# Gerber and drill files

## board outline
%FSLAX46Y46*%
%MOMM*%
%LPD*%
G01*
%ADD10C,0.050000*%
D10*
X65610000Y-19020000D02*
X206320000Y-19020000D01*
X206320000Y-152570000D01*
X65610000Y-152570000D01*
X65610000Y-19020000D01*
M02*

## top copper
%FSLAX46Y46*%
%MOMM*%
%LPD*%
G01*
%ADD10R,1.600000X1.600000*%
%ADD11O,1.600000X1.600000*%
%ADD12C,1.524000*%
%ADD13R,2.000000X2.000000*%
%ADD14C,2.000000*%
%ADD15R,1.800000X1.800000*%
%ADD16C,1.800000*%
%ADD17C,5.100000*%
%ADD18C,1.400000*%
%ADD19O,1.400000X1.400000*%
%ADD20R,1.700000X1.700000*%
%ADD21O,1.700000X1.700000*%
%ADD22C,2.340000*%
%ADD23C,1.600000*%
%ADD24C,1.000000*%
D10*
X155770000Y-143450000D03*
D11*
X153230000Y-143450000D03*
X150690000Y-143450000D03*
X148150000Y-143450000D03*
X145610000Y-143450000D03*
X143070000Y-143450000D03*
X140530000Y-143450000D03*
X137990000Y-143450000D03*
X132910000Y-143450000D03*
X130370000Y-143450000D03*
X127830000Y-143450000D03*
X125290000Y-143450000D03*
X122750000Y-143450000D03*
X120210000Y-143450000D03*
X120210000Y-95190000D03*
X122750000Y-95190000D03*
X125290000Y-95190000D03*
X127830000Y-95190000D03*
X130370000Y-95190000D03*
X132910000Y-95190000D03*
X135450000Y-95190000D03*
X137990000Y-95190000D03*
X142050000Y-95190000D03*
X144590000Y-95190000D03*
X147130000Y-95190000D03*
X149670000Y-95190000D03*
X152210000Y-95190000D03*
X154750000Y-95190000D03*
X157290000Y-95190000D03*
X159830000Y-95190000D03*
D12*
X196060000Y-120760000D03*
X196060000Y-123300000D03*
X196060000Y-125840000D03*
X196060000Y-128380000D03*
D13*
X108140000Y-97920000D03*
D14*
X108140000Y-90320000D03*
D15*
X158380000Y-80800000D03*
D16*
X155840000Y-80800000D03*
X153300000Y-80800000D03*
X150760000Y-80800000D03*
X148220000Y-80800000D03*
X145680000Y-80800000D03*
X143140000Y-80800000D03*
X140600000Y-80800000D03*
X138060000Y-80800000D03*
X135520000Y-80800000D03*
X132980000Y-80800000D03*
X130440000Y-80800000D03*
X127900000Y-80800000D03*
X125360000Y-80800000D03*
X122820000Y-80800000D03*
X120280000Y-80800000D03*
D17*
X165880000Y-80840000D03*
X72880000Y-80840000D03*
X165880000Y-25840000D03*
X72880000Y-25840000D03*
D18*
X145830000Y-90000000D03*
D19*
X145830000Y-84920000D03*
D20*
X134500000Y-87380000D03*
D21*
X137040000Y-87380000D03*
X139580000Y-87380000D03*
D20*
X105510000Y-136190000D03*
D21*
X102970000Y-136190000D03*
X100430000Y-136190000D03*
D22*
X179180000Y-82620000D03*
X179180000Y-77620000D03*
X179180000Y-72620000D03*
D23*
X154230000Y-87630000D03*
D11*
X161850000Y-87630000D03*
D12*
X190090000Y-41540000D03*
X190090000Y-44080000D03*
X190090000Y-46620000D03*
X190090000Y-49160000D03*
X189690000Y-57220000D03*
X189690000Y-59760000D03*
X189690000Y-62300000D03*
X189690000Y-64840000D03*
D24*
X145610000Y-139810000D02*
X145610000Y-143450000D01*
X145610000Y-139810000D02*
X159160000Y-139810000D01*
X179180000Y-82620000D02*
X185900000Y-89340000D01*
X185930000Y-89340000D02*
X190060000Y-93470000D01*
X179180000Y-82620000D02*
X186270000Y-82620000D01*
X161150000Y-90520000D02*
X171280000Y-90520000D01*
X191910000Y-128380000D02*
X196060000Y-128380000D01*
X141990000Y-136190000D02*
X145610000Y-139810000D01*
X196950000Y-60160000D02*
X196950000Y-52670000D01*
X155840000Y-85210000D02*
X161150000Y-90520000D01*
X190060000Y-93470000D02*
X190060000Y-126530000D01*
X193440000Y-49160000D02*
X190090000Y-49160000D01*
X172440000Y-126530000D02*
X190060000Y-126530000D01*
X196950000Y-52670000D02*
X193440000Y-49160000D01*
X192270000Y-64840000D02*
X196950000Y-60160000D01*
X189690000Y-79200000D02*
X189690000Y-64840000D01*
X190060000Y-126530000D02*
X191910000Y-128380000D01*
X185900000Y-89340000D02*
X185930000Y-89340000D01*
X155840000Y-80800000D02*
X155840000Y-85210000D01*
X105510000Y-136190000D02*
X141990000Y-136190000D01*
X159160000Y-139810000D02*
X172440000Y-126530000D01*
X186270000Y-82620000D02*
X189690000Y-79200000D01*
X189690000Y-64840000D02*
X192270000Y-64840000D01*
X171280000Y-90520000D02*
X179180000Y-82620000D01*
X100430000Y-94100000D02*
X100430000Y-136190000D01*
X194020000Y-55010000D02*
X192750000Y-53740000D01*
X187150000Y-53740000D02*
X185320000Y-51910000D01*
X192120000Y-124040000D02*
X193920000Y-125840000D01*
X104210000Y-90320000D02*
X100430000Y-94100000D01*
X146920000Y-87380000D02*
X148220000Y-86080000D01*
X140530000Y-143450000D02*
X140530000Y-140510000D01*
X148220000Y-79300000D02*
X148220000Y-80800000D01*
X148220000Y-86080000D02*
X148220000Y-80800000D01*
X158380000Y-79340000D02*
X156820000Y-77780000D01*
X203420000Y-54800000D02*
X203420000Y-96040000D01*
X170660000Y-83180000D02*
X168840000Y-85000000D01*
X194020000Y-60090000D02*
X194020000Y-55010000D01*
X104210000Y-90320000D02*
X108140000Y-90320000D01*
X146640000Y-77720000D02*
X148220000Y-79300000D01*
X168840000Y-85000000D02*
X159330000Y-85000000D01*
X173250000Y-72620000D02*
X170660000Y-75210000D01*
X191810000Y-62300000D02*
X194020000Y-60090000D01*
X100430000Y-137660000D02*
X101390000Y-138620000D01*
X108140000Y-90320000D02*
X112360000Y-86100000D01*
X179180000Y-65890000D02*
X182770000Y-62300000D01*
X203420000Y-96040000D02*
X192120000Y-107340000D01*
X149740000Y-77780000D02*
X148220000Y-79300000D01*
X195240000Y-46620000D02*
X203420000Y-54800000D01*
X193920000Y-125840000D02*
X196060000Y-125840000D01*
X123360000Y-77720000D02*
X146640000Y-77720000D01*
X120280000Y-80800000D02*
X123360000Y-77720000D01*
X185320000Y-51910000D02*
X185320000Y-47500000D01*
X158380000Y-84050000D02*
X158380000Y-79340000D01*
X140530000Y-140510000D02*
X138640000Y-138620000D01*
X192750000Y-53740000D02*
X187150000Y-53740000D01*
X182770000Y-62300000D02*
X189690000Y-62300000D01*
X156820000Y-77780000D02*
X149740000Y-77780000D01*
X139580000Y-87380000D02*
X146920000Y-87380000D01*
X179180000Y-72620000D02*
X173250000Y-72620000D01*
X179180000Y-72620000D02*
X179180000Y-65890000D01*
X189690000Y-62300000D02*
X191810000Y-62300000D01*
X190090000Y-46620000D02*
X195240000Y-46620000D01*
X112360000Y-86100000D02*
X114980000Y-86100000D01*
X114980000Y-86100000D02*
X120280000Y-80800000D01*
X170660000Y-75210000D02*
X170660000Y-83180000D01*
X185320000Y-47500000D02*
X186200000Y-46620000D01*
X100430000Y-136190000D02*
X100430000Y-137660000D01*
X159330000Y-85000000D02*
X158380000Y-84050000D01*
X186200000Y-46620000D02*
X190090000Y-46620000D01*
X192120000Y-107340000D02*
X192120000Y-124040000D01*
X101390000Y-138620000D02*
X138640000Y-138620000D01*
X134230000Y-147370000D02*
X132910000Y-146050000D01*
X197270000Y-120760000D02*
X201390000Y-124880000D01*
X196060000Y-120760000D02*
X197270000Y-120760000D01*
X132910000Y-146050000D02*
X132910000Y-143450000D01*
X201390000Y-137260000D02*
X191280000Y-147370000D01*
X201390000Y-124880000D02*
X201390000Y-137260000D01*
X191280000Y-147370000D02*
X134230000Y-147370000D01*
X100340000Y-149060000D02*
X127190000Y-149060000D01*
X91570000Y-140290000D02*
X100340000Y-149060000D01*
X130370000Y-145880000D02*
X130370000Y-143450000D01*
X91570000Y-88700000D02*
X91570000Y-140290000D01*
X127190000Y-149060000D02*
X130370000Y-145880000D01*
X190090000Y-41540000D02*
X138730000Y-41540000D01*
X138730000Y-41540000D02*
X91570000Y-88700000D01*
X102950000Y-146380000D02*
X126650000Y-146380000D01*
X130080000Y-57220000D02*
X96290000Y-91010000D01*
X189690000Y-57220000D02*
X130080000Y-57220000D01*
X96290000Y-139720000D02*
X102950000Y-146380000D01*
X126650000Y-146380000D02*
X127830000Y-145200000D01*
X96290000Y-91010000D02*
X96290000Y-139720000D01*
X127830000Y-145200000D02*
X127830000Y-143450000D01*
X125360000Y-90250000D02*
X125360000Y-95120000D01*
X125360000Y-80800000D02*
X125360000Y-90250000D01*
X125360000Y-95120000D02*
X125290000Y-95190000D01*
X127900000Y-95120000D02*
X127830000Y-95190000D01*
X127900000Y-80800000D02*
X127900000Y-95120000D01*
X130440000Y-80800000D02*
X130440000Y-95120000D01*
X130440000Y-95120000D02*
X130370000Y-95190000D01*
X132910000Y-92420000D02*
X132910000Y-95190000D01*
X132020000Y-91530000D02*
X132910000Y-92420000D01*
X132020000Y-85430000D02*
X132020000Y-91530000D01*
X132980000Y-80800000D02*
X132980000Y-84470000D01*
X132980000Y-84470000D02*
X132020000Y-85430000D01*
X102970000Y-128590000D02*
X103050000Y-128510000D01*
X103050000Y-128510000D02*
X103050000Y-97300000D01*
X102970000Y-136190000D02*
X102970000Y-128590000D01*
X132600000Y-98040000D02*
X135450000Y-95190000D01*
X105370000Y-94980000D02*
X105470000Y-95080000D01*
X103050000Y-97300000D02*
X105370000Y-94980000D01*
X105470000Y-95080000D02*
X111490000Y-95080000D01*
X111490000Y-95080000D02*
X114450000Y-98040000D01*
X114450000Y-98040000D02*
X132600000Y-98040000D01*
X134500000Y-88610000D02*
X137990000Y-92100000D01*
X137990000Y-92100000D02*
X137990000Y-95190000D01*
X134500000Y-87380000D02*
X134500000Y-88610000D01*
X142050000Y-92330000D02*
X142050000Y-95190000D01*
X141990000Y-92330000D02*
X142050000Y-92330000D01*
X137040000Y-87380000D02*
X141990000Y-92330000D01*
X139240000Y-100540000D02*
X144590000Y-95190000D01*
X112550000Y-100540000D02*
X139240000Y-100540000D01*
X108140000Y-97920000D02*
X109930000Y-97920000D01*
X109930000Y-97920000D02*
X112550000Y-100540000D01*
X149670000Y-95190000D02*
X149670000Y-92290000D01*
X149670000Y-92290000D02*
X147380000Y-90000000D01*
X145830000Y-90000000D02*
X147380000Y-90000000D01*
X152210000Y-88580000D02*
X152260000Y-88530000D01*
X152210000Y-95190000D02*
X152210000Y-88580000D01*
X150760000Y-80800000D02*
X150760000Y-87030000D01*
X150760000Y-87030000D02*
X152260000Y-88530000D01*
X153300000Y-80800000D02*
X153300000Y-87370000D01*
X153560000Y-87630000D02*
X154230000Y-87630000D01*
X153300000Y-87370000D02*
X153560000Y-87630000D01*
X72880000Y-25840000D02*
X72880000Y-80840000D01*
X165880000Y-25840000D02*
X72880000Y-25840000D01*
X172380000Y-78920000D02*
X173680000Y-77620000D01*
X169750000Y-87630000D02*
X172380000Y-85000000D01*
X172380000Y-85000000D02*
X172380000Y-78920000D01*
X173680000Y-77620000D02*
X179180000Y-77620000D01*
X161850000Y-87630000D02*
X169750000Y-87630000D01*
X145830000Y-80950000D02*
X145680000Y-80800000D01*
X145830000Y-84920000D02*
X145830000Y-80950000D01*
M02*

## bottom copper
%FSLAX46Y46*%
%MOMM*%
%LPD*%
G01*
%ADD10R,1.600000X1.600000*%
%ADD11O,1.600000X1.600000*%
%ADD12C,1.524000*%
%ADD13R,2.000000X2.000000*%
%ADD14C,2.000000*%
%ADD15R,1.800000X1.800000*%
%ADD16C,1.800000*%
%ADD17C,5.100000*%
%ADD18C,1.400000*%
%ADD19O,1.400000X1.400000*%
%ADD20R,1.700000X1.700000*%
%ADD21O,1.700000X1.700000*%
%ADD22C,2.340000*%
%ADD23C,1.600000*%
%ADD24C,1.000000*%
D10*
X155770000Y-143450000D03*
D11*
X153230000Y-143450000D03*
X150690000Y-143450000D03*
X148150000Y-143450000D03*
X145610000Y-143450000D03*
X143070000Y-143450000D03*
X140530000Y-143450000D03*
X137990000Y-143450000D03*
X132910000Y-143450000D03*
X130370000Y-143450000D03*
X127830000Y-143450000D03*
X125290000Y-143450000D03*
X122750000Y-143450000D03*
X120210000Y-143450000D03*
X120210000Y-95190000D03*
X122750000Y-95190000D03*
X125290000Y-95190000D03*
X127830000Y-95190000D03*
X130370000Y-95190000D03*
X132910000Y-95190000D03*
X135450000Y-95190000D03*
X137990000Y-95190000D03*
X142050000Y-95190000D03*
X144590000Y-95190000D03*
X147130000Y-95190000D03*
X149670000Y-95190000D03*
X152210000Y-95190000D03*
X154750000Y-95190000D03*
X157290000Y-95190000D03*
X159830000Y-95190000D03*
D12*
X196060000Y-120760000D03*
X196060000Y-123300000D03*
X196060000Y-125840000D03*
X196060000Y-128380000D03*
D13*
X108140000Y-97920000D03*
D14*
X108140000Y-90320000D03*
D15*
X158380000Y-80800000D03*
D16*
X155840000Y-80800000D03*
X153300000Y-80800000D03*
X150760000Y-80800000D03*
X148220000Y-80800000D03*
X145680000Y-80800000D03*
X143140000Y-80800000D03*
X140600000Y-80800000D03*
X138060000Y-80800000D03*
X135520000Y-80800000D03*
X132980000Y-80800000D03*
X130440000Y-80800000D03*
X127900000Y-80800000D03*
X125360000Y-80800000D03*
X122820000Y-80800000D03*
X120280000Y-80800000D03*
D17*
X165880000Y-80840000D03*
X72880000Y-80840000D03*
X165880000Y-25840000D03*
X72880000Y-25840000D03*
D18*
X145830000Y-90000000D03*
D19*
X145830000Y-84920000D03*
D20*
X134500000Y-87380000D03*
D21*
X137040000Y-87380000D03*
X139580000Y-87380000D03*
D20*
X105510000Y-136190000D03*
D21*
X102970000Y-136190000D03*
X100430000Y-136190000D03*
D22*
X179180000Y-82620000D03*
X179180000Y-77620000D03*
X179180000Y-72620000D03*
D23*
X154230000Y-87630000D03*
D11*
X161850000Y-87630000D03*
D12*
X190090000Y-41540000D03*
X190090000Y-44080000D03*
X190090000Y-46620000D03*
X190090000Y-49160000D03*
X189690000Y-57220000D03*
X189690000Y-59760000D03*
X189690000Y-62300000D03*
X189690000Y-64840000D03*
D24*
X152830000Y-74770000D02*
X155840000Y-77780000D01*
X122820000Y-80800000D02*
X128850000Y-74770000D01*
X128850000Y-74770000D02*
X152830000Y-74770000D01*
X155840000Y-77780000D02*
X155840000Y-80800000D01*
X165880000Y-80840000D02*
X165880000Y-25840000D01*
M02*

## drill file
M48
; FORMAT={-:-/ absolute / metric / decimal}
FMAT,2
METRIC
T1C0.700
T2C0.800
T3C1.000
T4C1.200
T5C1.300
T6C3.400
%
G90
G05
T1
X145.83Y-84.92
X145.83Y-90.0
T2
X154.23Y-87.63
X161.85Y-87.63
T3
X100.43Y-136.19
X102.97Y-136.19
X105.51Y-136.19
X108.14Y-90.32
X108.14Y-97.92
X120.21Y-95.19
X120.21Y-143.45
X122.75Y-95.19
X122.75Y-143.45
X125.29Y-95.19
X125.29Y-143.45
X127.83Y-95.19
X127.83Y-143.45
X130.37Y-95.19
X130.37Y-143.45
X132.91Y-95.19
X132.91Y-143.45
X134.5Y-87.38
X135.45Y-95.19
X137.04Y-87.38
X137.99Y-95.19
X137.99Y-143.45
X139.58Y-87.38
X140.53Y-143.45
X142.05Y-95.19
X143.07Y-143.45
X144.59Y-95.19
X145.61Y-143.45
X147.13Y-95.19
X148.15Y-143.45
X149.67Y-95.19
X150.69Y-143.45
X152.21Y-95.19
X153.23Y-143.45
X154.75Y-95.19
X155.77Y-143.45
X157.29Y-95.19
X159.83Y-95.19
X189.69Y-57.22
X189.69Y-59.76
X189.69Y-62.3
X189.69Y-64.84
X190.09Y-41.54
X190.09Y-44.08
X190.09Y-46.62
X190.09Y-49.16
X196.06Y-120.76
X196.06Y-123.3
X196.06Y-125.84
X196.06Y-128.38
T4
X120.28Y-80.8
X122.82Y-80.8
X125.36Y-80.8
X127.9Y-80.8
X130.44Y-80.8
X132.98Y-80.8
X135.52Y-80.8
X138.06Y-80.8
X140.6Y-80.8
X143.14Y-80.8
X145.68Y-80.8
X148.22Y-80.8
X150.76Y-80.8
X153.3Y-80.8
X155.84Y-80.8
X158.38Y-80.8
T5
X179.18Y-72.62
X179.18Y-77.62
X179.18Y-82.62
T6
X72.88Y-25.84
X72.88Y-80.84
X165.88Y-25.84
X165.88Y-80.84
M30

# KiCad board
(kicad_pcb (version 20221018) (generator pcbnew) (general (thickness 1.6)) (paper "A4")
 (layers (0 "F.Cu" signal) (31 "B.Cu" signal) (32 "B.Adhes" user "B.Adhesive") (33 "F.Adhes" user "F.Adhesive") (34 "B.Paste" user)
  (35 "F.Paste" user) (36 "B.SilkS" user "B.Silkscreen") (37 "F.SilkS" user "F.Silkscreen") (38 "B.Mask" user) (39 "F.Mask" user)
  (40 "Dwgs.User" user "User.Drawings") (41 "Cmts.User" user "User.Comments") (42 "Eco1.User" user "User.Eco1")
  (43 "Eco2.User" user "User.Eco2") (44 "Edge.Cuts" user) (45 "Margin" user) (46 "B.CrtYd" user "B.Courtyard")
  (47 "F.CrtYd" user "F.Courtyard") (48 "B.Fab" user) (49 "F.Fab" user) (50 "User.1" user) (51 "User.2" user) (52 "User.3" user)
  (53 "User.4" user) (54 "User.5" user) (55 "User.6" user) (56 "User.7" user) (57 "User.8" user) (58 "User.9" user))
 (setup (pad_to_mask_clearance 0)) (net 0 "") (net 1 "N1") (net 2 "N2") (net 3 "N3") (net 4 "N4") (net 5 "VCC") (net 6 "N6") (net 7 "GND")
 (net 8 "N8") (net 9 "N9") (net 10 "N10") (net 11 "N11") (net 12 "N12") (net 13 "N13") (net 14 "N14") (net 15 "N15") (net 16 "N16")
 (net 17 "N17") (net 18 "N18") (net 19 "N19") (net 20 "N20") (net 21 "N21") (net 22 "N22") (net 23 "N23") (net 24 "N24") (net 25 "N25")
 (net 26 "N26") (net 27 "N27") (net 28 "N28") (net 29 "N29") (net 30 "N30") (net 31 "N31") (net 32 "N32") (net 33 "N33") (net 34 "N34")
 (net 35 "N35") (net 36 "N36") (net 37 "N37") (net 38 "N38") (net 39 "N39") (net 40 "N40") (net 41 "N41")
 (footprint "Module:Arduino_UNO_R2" (layer "F.Cu") (at 155.77 143.45 180)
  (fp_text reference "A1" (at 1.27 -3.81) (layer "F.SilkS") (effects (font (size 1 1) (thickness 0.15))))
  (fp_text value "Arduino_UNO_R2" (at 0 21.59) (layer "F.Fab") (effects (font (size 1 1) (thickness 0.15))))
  (pad "1" thru_hole rect (at 0 0 270) (size 1.6 1.6) (drill 1) (layers "*.Cu" "*.Mask") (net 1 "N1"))
  (pad "2" thru_hole oval (at 2.54 0 270) (size 1.6 1.6) (drill 1) (layers "*.Cu" "*.Mask") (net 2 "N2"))
  (pad "3" thru_hole oval (at 5.08 0 270) (size 1.6 1.6) (drill 1) (layers "*.Cu" "*.Mask") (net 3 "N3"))
  (pad "4" thru_hole oval (at 7.62 0 270) (size 1.6 1.6) (drill 1) (layers "*.Cu" "*.Mask") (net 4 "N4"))
  (pad "5" thru_hole oval (at 10.16 0 270) (size 1.6 1.6) (drill 1) (layers "*.Cu" "*.Mask") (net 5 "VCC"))
  (pad "6" thru_hole oval (at 12.7 0 270) (size 1.6 1.6) (drill 1) (layers "*.Cu" "*.Mask") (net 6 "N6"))
  (pad "7" thru_hole oval (at 15.24 0 270) (size 1.6 1.6) (drill 1) (layers "*.Cu" "*.Mask") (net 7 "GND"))
  (pad "8" thru_hole oval (at 17.78 0 270) (size 1.6 1.6) (drill 1) (layers "*.Cu" "*.Mask") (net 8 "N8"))
  (pad "9" thru_hole oval (at 22.86 0 270) (size 1.6 1.6) (drill 1) (layers "*.Cu" "*.Mask") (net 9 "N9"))
  (pad "10" thru_hole oval (at 25.4 0 270) (size 1.6 1.6) (drill 1) (layers "*.Cu" "*.Mask") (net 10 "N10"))
  (pad "11" thru_hole oval (at 27.94 0 270) (size 1.6 1.6) (drill 1) (layers "*.Cu" "*.Mask") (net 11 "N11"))
  (pad "12" thru_hole oval (at 30.48 0 270) (size 1.6 1.6) (drill 1) (layers "*.Cu" "*.Mask") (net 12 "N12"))
  (pad "13" thru_hole oval (at 33.02 0 270) (size 1.6 1.6) (drill 1) (layers "*.Cu" "*.Mask") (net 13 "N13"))
  (pad "14" thru_hole oval (at 35.56 0 270) (size 1.6 1.6) (drill 1) (layers "*.Cu" "*.Mask") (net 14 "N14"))
  (pad "15" thru_hole oval (at 35.56 48.26 270) (size 1.6 1.6) (drill 1) (layers "*.Cu" "*.Mask") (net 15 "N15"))
  (pad "16" thru_hole oval (at 33.02 48.26 270) (size 1.6 1.6) (drill 1) (layers "*.Cu" "*.Mask") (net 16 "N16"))
  (pad "17" thru_hole oval (at 30.48 48.26 270) (size 1.6 1.6) (drill 1) (layers "*.Cu" "*.Mask") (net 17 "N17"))
  (pad "18" thru_hole oval (at 27.94 48.26 270) (size 1.6 1.6) (drill 1) (layers "*.Cu" "*.Mask") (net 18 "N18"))
  (pad "19" thru_hole oval (at 25.4 48.26 270) (size 1.6 1.6) (drill 1) (layers "*.Cu" "*.Mask") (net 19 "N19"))
  (pad "20" thru_hole oval (at 22.86 48.26 270) (size 1.6 1.6) (drill 1) (layers "*.Cu" "*.Mask") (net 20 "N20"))
  (pad "21" thru_hole oval (at 20.32 48.26 270) (size 1.6 1.6) (drill 1) (layers "*.Cu" "*.Mask") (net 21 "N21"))
  (pad "22" thru_hole oval (at 17.78 48.26 270) (size 1.6 1.6) (drill 1) (layers "*.Cu" "*.Mask") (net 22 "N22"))
  (pad "23" thru_hole oval (at 13.72 48.26 270) (size 1.6 1.6) (drill 1) (layers "*.Cu" "*.Mask") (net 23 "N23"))
  (pad "24" thru_hole oval (at 11.18 48.26 270) (size 1.6 1.6) (drill 1) (layers "*.Cu" "*.Mask") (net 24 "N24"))
  (pad "25" thru_hole oval (at 8.64 48.26 270) (size 1.6 1.6) (drill 1) (layers "*.Cu" "*.Mask") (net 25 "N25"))
  (pad "26" thru_hole oval (at 6.1 48.26 270) (size 1.6 1.6) (drill 1) (layers "*.Cu" "*.Mask") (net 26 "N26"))
  (pad "27" thru_hole oval (at 3.56 48.26 270) (size 1.6 1.6) (drill 1) (layers "*.Cu" "*.Mask") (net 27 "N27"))
  (pad "28" thru_hole oval (at 1.02 48.26 270) (size 1.6 1.6) (drill 1) (layers "*.Cu" "*.Mask") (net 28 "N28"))
  (pad "29" thru_hole oval (at -1.52 48.26 270) (size 1.6 1.6) (drill 1) (layers "*.Cu" "*.Mask") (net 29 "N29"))
  (pad "30" thru_hole oval (at -4.06 48.26 270) (size 1.6 1.6) (drill 1) (layers "*.Cu" "*.Mask") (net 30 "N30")))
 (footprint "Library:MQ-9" (layer "F.Cu") (at 201.14 115.68)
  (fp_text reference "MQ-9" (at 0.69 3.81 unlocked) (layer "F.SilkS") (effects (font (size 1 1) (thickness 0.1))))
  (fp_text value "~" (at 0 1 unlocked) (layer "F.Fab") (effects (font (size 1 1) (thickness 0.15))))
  (pad "1" thru_hole circle (at -5.08 5.08) (size 1.524 1.524) (drill 1) (layers "*.Cu" "*.Mask") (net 9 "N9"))
  (pad "2" thru_hole circle (at -5.08 7.62) (size 1.524 1.524) (drill 1) (layers "*.Cu" "*.Mask") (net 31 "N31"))
  (pad "3" thru_hole circle (at -5.08 10.16) (size 1.524 1.524) (drill 1) (layers "*.Cu" "*.Mask") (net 7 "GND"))
  (pad "4" thru_hole circle (at -5.08 12.7) (size 1.524 1.524) (drill 1) (layers "*.Cu" "*.Mask") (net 5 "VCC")))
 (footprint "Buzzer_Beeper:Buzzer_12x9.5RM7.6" (layer "F.Cu") (at 108.14 97.92 90)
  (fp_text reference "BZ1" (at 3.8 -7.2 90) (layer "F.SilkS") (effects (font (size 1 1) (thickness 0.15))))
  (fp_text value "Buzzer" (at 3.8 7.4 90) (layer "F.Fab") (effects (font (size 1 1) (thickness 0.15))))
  (pad "1" thru_hole rect (at 0 0 90) (size 2 2) (drill 1) (layers "*.Cu" "*.Mask") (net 24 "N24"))
  (pad "2" thru_hole circle (at 7.6 0 90) (size 2 2) (drill 1) (layers "*.Cu" "*.Mask") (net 7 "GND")))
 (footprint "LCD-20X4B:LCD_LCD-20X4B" (layer "F.Cu") (at 119.38 53.34 180)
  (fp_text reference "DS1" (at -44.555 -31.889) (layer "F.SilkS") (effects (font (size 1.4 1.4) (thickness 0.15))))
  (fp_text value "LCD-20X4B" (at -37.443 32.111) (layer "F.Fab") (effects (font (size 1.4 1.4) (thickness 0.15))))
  (pad "1" thru_hole rect (at -39 -27.46 180) (size 1.8 1.8) (drill 1.2) (layers "*.Cu" "*.Mask") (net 7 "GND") (solder_mask_margin 0.102))
  (pad "2" thru_hole circle (at -36.46 -27.46 180) (size 1.8 1.8) (drill 1.2) (layers "*.Cu" "*.Mask") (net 5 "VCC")
   (solder_mask_margin 0.102))
  (pad "3" thru_hole circle (at -33.92 -27.46 180) (size 1.8 1.8) (drill 1.2) (layers "*.Cu" "*.Mask") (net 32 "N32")
   (solder_mask_margin 0.102))
  (pad "4" thru_hole circle (at -31.38 -27.46 180) (size 1.8 1.8) (drill 1.2) (layers "*.Cu" "*.Mask") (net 27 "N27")
   (solder_mask_margin 0.102))
  (pad "5" thru_hole circle (at -28.84 -27.46 180) (size 1.8 1.8) (drill 1.2) (layers "*.Cu" "*.Mask") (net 7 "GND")
   (solder_mask_margin 0.102))
  (pad "6" thru_hole circle (at -26.3 -27.46 180) (size 1.8 1.8) (drill 1.2) (layers "*.Cu" "*.Mask") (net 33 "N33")
   (solder_mask_margin 0.102))
  (pad "7" thru_hole circle (at -23.76 -27.46 180) (size 1.8 1.8) (drill 1.2) (layers "*.Cu" "*.Mask") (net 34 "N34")
   (solder_mask_margin 0.102))
  (pad "8" thru_hole circle (at -21.22 -27.46 180) (size 1.8 1.8) (drill 1.2) (layers "*.Cu" "*.Mask") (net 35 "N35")
   (solder_mask_margin 0.102))
  (pad "9" thru_hole circle (at -18.68 -27.46 180) (size 1.8 1.8) (drill 1.2) (layers "*.Cu" "*.Mask") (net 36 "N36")
   (solder_mask_margin 0.102))
  (pad "10" thru_hole circle (at -16.14 -27.46 180) (size 1.8 1.8) (drill 1.2) (layers "*.Cu" "*.Mask") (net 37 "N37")
   (solder_mask_margin 0.102))
  (pad "11" thru_hole circle (at -13.6 -27.46 180) (size 1.8 1.8) (drill 1.2) (layers "*.Cu" "*.Mask") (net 20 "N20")
   (solder_mask_margin 0.102))
  (pad "12" thru_hole circle (at -11.06 -27.46 180) (size 1.8 1.8) (drill 1.2) (layers "*.Cu" "*.Mask") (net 19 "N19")
   (solder_mask_margin 0.102))
  (pad "13" thru_hole circle (at -8.52 -27.46 180) (size 1.8 1.8) (drill 1.2) (layers "*.Cu" "*.Mask") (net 18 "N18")
   (solder_mask_margin 0.102))
  (pad "14" thru_hole circle (at -5.98 -27.46 180) (size 1.8 1.8) (drill 1.2) (layers "*.Cu" "*.Mask") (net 17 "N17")
   (solder_mask_margin 0.102))
  (pad "15" thru_hole circle (at -3.44 -27.46 180) (size 1.8 1.8) (drill 1.2) (layers "*.Cu" "*.Mask") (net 5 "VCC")
   (solder_mask_margin 0.102))
  (pad "16" thru_hole circle (at -0.9 -27.46 180) (size 1.8 1.8) (drill 1.2) (layers "*.Cu" "*.Mask") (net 7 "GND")
   (solder_mask_margin 0.102))
  (pad "S1" thru_hole circle (at -46.5 -27.5 180) (size 5.1 5.1) (drill 3.4) (layers "*.Cu" "*.Mask") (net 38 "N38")
   (solder_mask_margin 0.102))
  (pad "S2" thru_hole circle (at 46.5 -27.5 180) (size 5.1 5.1) (drill 3.4) (layers "*.Cu" "*.Mask") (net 38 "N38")
   (solder_mask_margin 0.102))
  (pad "S3" thru_hole circle (at -46.5 27.5 180) (size 5.1 5.1) (drill 3.4) (layers "*.Cu" "*.Mask") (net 38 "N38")
   (solder_mask_margin 0.102))
  (pad "S4" thru_hole circle (at 46.5 27.5 180) (size 5.1 5.1) (drill 3.4) (layers "*.Cu" "*.Mask") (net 38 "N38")
   (solder_mask_margin 0.102)))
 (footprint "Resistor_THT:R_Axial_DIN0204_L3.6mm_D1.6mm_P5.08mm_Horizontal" (layer "F.Cu") (at 145.83 90 90)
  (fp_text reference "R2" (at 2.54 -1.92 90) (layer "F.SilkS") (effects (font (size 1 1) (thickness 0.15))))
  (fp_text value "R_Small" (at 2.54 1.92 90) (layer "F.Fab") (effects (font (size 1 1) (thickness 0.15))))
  (pad "1" thru_hole circle (at 0 0 90) (size 1.4 1.4) (drill 0.7) (layers "*.Cu" "*.Mask") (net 26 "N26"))
  (pad "2" thru_hole oval (at 5.08 0 90) (size 1.4 1.4) (drill 0.7) (layers "*.Cu" "*.Mask") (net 33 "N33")))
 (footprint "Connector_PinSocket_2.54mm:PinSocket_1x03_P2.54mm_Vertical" (layer "F.Cu") (at 134.5 87.38 90)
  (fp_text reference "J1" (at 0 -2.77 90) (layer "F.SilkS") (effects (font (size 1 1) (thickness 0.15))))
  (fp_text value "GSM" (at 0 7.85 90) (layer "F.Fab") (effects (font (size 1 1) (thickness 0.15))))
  (pad "1" thru_hole rect (at 0 0 90) (size 1.7 1.7) (drill 1) (layers "*.Cu" "*.Mask") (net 22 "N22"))
  (pad "2" thru_hole oval (at 0 2.54 90) (size 1.7 1.7) (drill 1) (layers "*.Cu" "*.Mask") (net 23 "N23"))
  (pad "3" thru_hole oval (at 0 5.08 90) (size 1.7 1.7) (drill 1) (layers "*.Cu" "*.Mask") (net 7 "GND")))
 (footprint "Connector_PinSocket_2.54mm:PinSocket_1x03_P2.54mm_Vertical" (layer "F.Cu") (at 105.51 136.19 -90)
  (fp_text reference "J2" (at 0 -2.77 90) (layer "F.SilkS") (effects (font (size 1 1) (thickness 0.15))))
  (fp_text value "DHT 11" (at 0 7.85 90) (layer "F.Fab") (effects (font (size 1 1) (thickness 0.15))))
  (pad "1" thru_hole rect (at 0 0 270) (size 1.7 1.7) (drill 1) (layers "*.Cu" "*.Mask") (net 5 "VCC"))
  (pad "2" thru_hole oval (at 0 2.54 270) (size 1.7 1.7) (drill 1) (layers "*.Cu" "*.Mask") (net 21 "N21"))
  (pad "3" thru_hole oval (at 0 5.08 270) (size 1.7 1.7) (drill 1) (layers "*.Cu" "*.Mask") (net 7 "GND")))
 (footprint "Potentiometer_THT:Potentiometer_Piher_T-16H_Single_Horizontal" (layer "F.Cu") (at 179.18 82.62)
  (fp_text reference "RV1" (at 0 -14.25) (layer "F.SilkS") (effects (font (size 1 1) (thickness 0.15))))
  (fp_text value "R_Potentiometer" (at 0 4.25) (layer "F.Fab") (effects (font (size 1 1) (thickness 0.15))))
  (pad "1" thru_hole circle (at 0 0) (size 2.34 2.34) (drill 1.3) (layers "*.Cu" "*.Mask") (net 5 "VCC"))
  (pad "2" thru_hole circle (at 0 -5) (size 2.34 2.34) (drill 1.3) (layers "*.Cu" "*.Mask") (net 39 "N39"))
  (pad "3" thru_hole circle (at 0 -10) (size 2.34 2.34) (drill 1.3) (layers "*.Cu" "*.Mask") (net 7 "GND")))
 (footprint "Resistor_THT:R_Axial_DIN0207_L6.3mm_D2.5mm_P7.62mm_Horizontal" (layer "F.Cu") (at 154.23 87.63)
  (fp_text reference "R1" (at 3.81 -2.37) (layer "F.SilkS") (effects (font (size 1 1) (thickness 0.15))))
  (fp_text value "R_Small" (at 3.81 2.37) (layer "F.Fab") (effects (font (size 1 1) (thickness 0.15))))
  (pad "1" thru_hole circle (at 0 0) (size 1.6 1.6) (drill 0.8) (layers "*.Cu" "*.Mask") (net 32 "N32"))
  (pad "2" thru_hole oval (at 7.62 0) (size 1.6 1.6) (drill 0.8) (layers "*.Cu" "*.Mask") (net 39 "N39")))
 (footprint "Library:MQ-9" (layer "F.Cu") (at 195.17 36.46)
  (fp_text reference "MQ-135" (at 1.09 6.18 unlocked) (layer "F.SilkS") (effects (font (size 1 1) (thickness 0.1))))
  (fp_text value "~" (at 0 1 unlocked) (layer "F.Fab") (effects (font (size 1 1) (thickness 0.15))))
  (pad "1" thru_hole circle (at -5.08 5.08) (size 1.524 1.524) (drill 1) (layers "*.Cu" "*.Mask") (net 10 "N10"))
  (pad "2" thru_hole circle (at -5.08 7.62) (size 1.524 1.524) (drill 1) (layers "*.Cu" "*.Mask") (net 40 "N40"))
  (pad "3" thru_hole circle (at -5.08 10.16) (size 1.524 1.524) (drill 1) (layers "*.Cu" "*.Mask") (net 7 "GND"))
  (pad "4" thru_hole circle (at -5.08 12.7) (size 1.524 1.524) (drill 1) (layers "*.Cu" "*.Mask") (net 5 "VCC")))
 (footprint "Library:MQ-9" (layer "F.Cu") (at 194.77 52.14)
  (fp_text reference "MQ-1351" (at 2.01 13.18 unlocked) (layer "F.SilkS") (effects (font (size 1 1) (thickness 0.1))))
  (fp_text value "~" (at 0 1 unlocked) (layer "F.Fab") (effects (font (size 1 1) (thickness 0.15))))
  (pad "1" thru_hole circle (at -5.08 5.08) (size 1.524 1.524) (drill 1) (layers "*.Cu" "*.Mask") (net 11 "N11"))
  (pad "2" thru_hole circle (at -5.08 7.62) (size 1.524 1.524) (drill 1) (layers "*.Cu" "*.Mask") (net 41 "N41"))
  (pad "3" thru_hole circle (at -5.08 10.16) (size 1.524 1.524) (drill 1) (layers "*.Cu" "*.Mask") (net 7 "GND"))
  (pad "4" thru_hole circle (at -5.08 12.7) (size 1.524 1.524) (drill 1) (layers "*.Cu" "*.Mask") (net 5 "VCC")))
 (gr_rect (start 65.61 19.02) (end 206.32 152.57) (stroke (width 0.05) (type default)) (fill none) (layer "Edge.Cuts"))
 (segment (start 145.61 139.81) (end 145.61 143.45) (width 1) (layer "F.Cu") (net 5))
 (segment (start 145.61 139.81) (end 159.16 139.81) (width 1) (layer "F.Cu") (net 5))
 (segment (start 179.18 82.62) (end 185.9 89.34) (width 1) (layer "F.Cu") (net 5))
 (segment (start 185.93 89.34) (end 190.06 93.47) (width 1) (layer "F.Cu") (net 5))
 (segment (start 179.18 82.62) (end 186.27 82.62) (width 1) (layer "F.Cu") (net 5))
 (segment (start 161.15 90.52) (end 171.28 90.52) (width 1) (layer "F.Cu") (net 5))
 (segment (start 191.91 128.38) (end 196.06 128.38) (width 1) (layer "F.Cu") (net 5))
 (segment (start 141.99 136.19) (end 145.61 139.81) (width 1) (layer "F.Cu") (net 5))
 (segment (start 196.95 60.16) (end 196.95 52.67) (width 1) (layer "F.Cu") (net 5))
 (segment (start 155.84 85.21) (end 161.15 90.52) (width 1) (layer "F.Cu") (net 5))
 (segment (start 190.06 93.47) (end 190.06 126.53) (width 1) (layer "F.Cu") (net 5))
 (segment (start 193.44 49.16) (end 190.09 49.16) (width 1) (layer "F.Cu") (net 5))
 (segment (start 172.44 126.53) (end 190.06 126.53) (width 1) (layer "F.Cu") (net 5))
 (segment (start 196.95 52.67) (end 193.44 49.16) (width 1) (layer "F.Cu") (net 5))
 (segment (start 192.27 64.84) (end 196.95 60.16) (width 1) (layer "F.Cu") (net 5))
 (segment (start 189.69 79.2) (end 189.69 64.84) (width 1) (layer "F.Cu") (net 5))
 (segment (start 190.06 126.53) (end 191.91 128.38) (width 1) (layer "F.Cu") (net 5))
 (segment (start 185.9 89.34) (end 185.93 89.34) (width 1) (layer "F.Cu") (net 5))
 (segment (start 155.84 80.8) (end 155.84 85.21) (width 1) (layer "F.Cu") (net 5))
 (segment (start 105.51 136.19) (end 141.99 136.19) (width 1) (layer "F.Cu") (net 5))
 (segment (start 159.16 139.81) (end 172.44 126.53) (width 1) (layer "F.Cu") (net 5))
 (segment (start 186.27 82.62) (end 189.69 79.2) (width 1) (layer "F.Cu") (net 5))
 (segment (start 189.69 64.84) (end 192.27 64.84) (width 1) (layer "F.Cu") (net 5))
 (segment (start 171.28 90.52) (end 179.18 82.62) (width 1) (layer "F.Cu") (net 5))
 (segment (start 152.83 74.77) (end 155.84 77.78) (width 1) (layer "B.Cu") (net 5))
 (segment (start 122.82 80.8) (end 128.85 74.77) (width 1) (layer "B.Cu") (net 5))
 (segment (start 128.85 74.77) (end 152.83 74.77) (width 1) (layer "B.Cu") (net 5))
 (segment (start 155.84 77.78) (end 155.84 80.8) (width 1) (layer "B.Cu") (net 5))
 (segment (start 100.43 94.1) (end 100.43 136.19) (width 1) (layer "F.Cu") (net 7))
 (segment (start 194.02 55.01) (end 192.75 53.74) (width 1) (layer "F.Cu") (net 7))
 (segment (start 187.15 53.74) (end 185.32 51.91) (width 1) (layer "F.Cu") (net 7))
 (segment (start 192.12 124.04) (end 193.92 125.84) (width 1) (layer "F.Cu") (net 7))
 (segment (start 104.21 90.32) (end 100.43 94.1) (width 1) (layer "F.Cu") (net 7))
 (segment (start 146.92 87.38) (end 148.22 86.08) (width 1) (layer "F.Cu") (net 7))
 (segment (start 140.53 143.45) (end 140.53 140.51) (width 1) (layer "F.Cu") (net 7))
 (segment (start 148.22 79.3) (end 148.22 80.8) (width 1) (layer "F.Cu") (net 7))
 (segment (start 148.22 86.08) (end 148.22 80.8) (width 1) (layer "F.Cu") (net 7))
 (segment (start 158.38 79.34) (end 156.82 77.78) (width 1) (layer "F.Cu") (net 7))
 (segment (start 203.42 54.8) (end 203.42 96.04) (width 1) (layer "F.Cu") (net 7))
 (segment (start 170.66 83.18) (end 168.84 85) (width 1) (layer "F.Cu") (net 7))
 (segment (start 194.02 60.09) (end 194.02 55.01) (width 1) (layer "F.Cu") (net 7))
 (segment (start 104.21 90.32) (end 108.14 90.32) (width 1) (layer "F.Cu") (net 7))
 (segment (start 146.64 77.72) (end 148.22 79.3) (width 1) (layer "F.Cu") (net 7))
 (segment (start 168.84 85) (end 159.33 85) (width 1) (layer "F.Cu") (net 7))
 (segment (start 173.25 72.62) (end 170.66 75.21) (width 1) (layer "F.Cu") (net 7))
 (segment (start 191.81 62.3) (end 194.02 60.09) (width 1) (layer "F.Cu") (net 7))
 (segment (start 100.43 137.66) (end 101.39 138.62) (width 1) (layer "F.Cu") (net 7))
 (segment (start 108.14 90.32) (end 112.36 86.1) (width 1) (layer "F.Cu") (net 7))
 (segment (start 179.18 65.89) (end 182.77 62.3) (width 1) (layer "F.Cu") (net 7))
 (segment (start 203.42 96.04) (end 192.12 107.34) (width 1) (layer "F.Cu") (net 7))
 (segment (start 149.74 77.78) (end 148.22 79.3) (width 1) (layer "F.Cu") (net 7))
 (segment (start 195.24 46.62) (end 203.42 54.8) (width 1) (layer "F.Cu") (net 7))
 (segment (start 193.92 125.84) (end 196.06 125.84) (width 1) (layer "F.Cu") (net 7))
 (segment (start 123.36 77.72) (end 146.64 77.72) (width 1) (layer "F.Cu") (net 7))
 (segment (start 120.28 80.8) (end 123.36 77.72) (width 1) (layer "F.Cu") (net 7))
 (segment (start 185.32 51.91) (end 185.32 47.5) (width 1) (layer "F.Cu") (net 7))
 (segment (start 158.38 84.05) (end 158.38 79.34) (width 1) (layer "F.Cu") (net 7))
 (segment (start 140.53 140.51) (end 138.64 138.62) (width 1) (layer "F.Cu") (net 7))
 (segment (start 192.75 53.74) (end 187.15 53.74) (width 1) (layer "F.Cu") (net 7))
 (segment (start 182.77 62.3) (end 189.69 62.3) (width 1) (layer "F.Cu") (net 7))
 (segment (start 156.82 77.78) (end 149.74 77.78) (width 1) (layer "F.Cu") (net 7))
 (segment (start 139.58 87.38) (end 146.92 87.38) (width 1) (layer "F.Cu") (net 7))
 (segment (start 179.18 72.62) (end 173.25 72.62) (width 1) (layer "F.Cu") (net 7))
 (segment (start 179.18 72.62) (end 179.18 65.89) (width 1) (layer "F.Cu") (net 7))
 (segment (start 189.69 62.3) (end 191.81 62.3) (width 1) (layer "F.Cu") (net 7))
 (segment (start 190.09 46.62) (end 195.24 46.62) (width 1) (layer "F.Cu") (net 7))
 (segment (start 112.36 86.1) (end 114.98 86.1) (width 1) (layer "F.Cu") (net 7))
 (segment (start 114.98 86.1) (end 120.28 80.8) (width 1) (layer "F.Cu") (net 7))
 (segment (start 170.66 75.21) (end 170.66 83.18) (width 1) (layer "F.Cu") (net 7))
 (segment (start 185.32 47.5) (end 186.2 46.62) (width 1) (layer "F.Cu") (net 7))
 (segment (start 100.43 136.19) (end 100.43 137.66) (width 1) (layer "F.Cu") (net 7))
 (segment (start 159.33 85) (end 158.38 84.05) (width 1) (layer "F.Cu") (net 7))
 (segment (start 186.2 46.62) (end 190.09 46.62) (width 1) (layer "F.Cu") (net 7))
 (segment (start 192.12 107.34) (end 192.12 124.04) (width 1) (layer "F.Cu") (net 7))
 (segment (start 101.39 138.62) (end 138.64 138.62) (width 1) (layer "F.Cu") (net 7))
 (segment (start 134.23 147.37) (end 132.91 146.05) (width 1) (layer "F.Cu") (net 9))
 (segment (start 197.27 120.76) (end 201.39 124.88) (width 1) (layer "F.Cu") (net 9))
 (segment (start 196.06 120.76) (end 197.27 120.76) (width 1) (layer "F.Cu") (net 9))
 (segment (start 132.91 146.05) (end 132.91 143.45) (width 1) (layer "F.Cu") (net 9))
 (segment (start 201.39 137.26) (end 191.28 147.37) (width 1) (layer "F.Cu") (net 9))
 (segment (start 201.39 124.88) (end 201.39 137.26) (width 1) (layer "F.Cu") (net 9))
 (segment (start 191.28 147.37) (end 134.23 147.37) (width 1) (layer "F.Cu") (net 9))
 (segment (start 100.34 149.06) (end 127.19 149.06) (width 1) (layer "F.Cu") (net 10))
 (segment (start 91.57 140.29) (end 100.34 149.06) (width 1) (layer "F.Cu") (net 10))
 (segment (start 130.37 145.88) (end 130.37 143.45) (width 1) (layer "F.Cu") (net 10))
 (segment (start 91.57 88.7) (end 91.57 140.29) (width 1) (layer "F.Cu") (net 10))
 (segment (start 127.19 149.06) (end 130.37 145.88) (width 1) (layer "F.Cu") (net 10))
 (segment (start 190.09 41.54) (end 138.73 41.54) (width 1) (layer "F.Cu") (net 10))
 (segment (start 138.73 41.54) (end 91.57 88.7) (width 1) (layer "F.Cu") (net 10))
 (segment (start 102.95 146.38) (end 126.65 146.38) (width 1) (layer "F.Cu") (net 11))
 (segment (start 130.08 57.22) (end 96.29 91.01) (width 1) (layer "F.Cu") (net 11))
 (segment (start 189.69 57.22) (end 130.08 57.22) (width 1) (layer "F.Cu") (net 11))
 (segment (start 96.29 139.72) (end 102.95 146.38) (width 1) (layer "F.Cu") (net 11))
 (segment (start 126.65 146.38) (end 127.83 145.2) (width 1) (layer "F.Cu") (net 11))
 (segment (start 96.29 91.01) (end 96.29 139.72) (width 1) (layer "F.Cu") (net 11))
 (segment (start 127.83 145.2) (end 127.83 143.45) (width 1) (layer "F.Cu") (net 11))
 (segment (start 125.36 90.25) (end 125.36 95.12) (width 1) (layer "F.Cu") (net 17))
 (segment (start 125.36 80.8) (end 125.36 90.25) (width 1) (layer "F.Cu") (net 17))
 (segment (start 125.36 95.12) (end 125.29 95.19) (width 1) (layer "F.Cu") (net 17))
 (segment (start 127.9 95.12) (end 127.83 95.19) (width 1) (layer "F.Cu") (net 18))
 (segment (start 127.9 80.8) (end 127.9 95.12) (width 1) (layer "F.Cu") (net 18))
 (segment (start 130.44 80.8) (end 130.44 95.12) (width 1) (layer "F.Cu") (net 19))
 (segment (start 130.44 95.12) (end 130.37 95.19) (width 1) (layer "F.Cu") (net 19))
 (segment (start 132.91 92.42) (end 132.91 95.19) (width 1) (layer "F.Cu") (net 20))
 (segment (start 132.02 91.53) (end 132.91 92.42) (width 1) (layer "F.Cu") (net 20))
 (segment (start 132.02 85.43) (end 132.02 91.53) (width 1) (layer "F.Cu") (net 20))
 (segment (start 132.98 80.8) (end 132.98 84.47) (width 1) (layer "F.Cu") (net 20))
 (segment (start 132.98 84.47) (end 132.02 85.43) (width 1) (layer "F.Cu") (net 20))
 (segment (start 102.97 128.59) (end 103.05 128.51) (width 1) (layer "F.Cu") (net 21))
 (segment (start 103.05 128.51) (end 103.05 97.3) (width 1) (layer "F.Cu") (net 21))
 (segment (start 102.97 136.19) (end 102.97 128.59) (width 1) (layer "F.Cu") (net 21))
 (segment (start 132.6 98.04) (end 135.45 95.19) (width 1) (layer "F.Cu") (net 21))
 (segment (start 105.37 94.98) (end 105.47 95.08) (width 1) (layer "F.Cu") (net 21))
 (segment (start 103.05 97.3) (end 105.37 94.98) (width 1) (layer "F.Cu") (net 21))
 (segment (start 105.47 95.08) (end 111.49 95.08) (width 1) (layer "F.Cu") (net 21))
 (segment (start 111.49 95.08) (end 114.45 98.04) (width 1) (layer "F.Cu") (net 21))
 (segment (start 114.45 98.04) (end 132.6 98.04) (width 1) (layer "F.Cu") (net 21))
 (segment (start 134.5 88.61) (end 137.99 92.1) (width 1) (layer "F.Cu") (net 22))
 (segment (start 137.99 92.1) (end 137.99 95.19) (width 1) (layer "F.Cu") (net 22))
 (segment (start 134.5 87.38) (end 134.5 88.61) (width 1) (layer "F.Cu") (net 22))
 (segment (start 142.05 92.33) (end 142.05 95.19) (width 1) (layer "F.Cu") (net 23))
 (segment (start 141.99 92.33) (end 142.05 92.33) (width 1) (layer "F.Cu") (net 23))
 (segment (start 137.04 87.38) (end 141.99 92.33) (width 1) (layer "F.Cu") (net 23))
 (segment (start 139.24 100.54) (end 144.59 95.19) (width 1) (layer "F.Cu") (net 24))
 (segment (start 112.55 100.54) (end 139.24 100.54) (width 1) (layer "F.Cu") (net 24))
 (segment (start 108.14 97.92) (end 109.93 97.92) (width 1) (layer "F.Cu") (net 24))
 (segment (start 109.93 97.92) (end 112.55 100.54) (width 1) (layer "F.Cu") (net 24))
 (segment (start 149.67 95.19) (end 149.67 92.29) (width 1) (layer "F.Cu") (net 26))
 (segment (start 149.67 92.29) (end 147.38 90) (width 1) (layer "F.Cu") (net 26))
 (segment (start 145.83 90) (end 147.38 90) (width 1) (layer "F.Cu") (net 26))
 (segment (start 152.21 88.58) (end 152.26 88.53) (width 1) (layer "F.Cu") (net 27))
 (segment (start 152.21 95.19) (end 152.21 88.58) (width 1) (layer "F.Cu") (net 27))
 (segment (start 150.76 80.8) (end 150.76 87.03) (width 1) (layer "F.Cu") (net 27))
 (segment (start 150.76 87.03) (end 152.26 88.53) (width 1) (layer "F.Cu") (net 27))
 (segment (start 153.3 80.8) (end 153.3 87.37) (width 1) (layer "F.Cu") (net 32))
 (segment (start 153.56 87.63) (end 154.23 87.63) (width 1) (layer "F.Cu") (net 32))
 (segment (start 153.3 87.37) (end 153.56 87.63) (width 1) (layer "F.Cu") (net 32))
 (segment (start 72.88 25.84) (end 72.88 80.84) (width 1) (layer "F.Cu") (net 38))
 (segment (start 165.88 25.84) (end 72.88 25.84) (width 1) (layer "F.Cu") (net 38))
 (segment (start 165.88 80.84) (end 165.88 25.84) (width 1) (layer "B.Cu") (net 38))
 (segment (start 172.38 78.92) (end 173.68 77.62) (width 1) (layer "F.Cu") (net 39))
 (segment (start 169.75 87.63) (end 172.38 85) (width 1) (layer "F.Cu") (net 39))
 (segment (start 172.38 85) (end 172.38 78.92) (width 1) (layer "F.Cu") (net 39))
 (segment (start 173.68 77.62) (end 179.18 77.62) (width 1) (layer "F.Cu") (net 39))
 (segment (start 161.85 87.63) (end 169.75 87.63) (width 1) (layer "F.Cu") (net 39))
 (segment (start 145.83 80.95) (end 145.68 80.8) (width 1) (layer "F.Cu") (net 33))
 (segment (start 145.83 84.92) (end 145.83 80.95) (width 1) (layer "F.Cu") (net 33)))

